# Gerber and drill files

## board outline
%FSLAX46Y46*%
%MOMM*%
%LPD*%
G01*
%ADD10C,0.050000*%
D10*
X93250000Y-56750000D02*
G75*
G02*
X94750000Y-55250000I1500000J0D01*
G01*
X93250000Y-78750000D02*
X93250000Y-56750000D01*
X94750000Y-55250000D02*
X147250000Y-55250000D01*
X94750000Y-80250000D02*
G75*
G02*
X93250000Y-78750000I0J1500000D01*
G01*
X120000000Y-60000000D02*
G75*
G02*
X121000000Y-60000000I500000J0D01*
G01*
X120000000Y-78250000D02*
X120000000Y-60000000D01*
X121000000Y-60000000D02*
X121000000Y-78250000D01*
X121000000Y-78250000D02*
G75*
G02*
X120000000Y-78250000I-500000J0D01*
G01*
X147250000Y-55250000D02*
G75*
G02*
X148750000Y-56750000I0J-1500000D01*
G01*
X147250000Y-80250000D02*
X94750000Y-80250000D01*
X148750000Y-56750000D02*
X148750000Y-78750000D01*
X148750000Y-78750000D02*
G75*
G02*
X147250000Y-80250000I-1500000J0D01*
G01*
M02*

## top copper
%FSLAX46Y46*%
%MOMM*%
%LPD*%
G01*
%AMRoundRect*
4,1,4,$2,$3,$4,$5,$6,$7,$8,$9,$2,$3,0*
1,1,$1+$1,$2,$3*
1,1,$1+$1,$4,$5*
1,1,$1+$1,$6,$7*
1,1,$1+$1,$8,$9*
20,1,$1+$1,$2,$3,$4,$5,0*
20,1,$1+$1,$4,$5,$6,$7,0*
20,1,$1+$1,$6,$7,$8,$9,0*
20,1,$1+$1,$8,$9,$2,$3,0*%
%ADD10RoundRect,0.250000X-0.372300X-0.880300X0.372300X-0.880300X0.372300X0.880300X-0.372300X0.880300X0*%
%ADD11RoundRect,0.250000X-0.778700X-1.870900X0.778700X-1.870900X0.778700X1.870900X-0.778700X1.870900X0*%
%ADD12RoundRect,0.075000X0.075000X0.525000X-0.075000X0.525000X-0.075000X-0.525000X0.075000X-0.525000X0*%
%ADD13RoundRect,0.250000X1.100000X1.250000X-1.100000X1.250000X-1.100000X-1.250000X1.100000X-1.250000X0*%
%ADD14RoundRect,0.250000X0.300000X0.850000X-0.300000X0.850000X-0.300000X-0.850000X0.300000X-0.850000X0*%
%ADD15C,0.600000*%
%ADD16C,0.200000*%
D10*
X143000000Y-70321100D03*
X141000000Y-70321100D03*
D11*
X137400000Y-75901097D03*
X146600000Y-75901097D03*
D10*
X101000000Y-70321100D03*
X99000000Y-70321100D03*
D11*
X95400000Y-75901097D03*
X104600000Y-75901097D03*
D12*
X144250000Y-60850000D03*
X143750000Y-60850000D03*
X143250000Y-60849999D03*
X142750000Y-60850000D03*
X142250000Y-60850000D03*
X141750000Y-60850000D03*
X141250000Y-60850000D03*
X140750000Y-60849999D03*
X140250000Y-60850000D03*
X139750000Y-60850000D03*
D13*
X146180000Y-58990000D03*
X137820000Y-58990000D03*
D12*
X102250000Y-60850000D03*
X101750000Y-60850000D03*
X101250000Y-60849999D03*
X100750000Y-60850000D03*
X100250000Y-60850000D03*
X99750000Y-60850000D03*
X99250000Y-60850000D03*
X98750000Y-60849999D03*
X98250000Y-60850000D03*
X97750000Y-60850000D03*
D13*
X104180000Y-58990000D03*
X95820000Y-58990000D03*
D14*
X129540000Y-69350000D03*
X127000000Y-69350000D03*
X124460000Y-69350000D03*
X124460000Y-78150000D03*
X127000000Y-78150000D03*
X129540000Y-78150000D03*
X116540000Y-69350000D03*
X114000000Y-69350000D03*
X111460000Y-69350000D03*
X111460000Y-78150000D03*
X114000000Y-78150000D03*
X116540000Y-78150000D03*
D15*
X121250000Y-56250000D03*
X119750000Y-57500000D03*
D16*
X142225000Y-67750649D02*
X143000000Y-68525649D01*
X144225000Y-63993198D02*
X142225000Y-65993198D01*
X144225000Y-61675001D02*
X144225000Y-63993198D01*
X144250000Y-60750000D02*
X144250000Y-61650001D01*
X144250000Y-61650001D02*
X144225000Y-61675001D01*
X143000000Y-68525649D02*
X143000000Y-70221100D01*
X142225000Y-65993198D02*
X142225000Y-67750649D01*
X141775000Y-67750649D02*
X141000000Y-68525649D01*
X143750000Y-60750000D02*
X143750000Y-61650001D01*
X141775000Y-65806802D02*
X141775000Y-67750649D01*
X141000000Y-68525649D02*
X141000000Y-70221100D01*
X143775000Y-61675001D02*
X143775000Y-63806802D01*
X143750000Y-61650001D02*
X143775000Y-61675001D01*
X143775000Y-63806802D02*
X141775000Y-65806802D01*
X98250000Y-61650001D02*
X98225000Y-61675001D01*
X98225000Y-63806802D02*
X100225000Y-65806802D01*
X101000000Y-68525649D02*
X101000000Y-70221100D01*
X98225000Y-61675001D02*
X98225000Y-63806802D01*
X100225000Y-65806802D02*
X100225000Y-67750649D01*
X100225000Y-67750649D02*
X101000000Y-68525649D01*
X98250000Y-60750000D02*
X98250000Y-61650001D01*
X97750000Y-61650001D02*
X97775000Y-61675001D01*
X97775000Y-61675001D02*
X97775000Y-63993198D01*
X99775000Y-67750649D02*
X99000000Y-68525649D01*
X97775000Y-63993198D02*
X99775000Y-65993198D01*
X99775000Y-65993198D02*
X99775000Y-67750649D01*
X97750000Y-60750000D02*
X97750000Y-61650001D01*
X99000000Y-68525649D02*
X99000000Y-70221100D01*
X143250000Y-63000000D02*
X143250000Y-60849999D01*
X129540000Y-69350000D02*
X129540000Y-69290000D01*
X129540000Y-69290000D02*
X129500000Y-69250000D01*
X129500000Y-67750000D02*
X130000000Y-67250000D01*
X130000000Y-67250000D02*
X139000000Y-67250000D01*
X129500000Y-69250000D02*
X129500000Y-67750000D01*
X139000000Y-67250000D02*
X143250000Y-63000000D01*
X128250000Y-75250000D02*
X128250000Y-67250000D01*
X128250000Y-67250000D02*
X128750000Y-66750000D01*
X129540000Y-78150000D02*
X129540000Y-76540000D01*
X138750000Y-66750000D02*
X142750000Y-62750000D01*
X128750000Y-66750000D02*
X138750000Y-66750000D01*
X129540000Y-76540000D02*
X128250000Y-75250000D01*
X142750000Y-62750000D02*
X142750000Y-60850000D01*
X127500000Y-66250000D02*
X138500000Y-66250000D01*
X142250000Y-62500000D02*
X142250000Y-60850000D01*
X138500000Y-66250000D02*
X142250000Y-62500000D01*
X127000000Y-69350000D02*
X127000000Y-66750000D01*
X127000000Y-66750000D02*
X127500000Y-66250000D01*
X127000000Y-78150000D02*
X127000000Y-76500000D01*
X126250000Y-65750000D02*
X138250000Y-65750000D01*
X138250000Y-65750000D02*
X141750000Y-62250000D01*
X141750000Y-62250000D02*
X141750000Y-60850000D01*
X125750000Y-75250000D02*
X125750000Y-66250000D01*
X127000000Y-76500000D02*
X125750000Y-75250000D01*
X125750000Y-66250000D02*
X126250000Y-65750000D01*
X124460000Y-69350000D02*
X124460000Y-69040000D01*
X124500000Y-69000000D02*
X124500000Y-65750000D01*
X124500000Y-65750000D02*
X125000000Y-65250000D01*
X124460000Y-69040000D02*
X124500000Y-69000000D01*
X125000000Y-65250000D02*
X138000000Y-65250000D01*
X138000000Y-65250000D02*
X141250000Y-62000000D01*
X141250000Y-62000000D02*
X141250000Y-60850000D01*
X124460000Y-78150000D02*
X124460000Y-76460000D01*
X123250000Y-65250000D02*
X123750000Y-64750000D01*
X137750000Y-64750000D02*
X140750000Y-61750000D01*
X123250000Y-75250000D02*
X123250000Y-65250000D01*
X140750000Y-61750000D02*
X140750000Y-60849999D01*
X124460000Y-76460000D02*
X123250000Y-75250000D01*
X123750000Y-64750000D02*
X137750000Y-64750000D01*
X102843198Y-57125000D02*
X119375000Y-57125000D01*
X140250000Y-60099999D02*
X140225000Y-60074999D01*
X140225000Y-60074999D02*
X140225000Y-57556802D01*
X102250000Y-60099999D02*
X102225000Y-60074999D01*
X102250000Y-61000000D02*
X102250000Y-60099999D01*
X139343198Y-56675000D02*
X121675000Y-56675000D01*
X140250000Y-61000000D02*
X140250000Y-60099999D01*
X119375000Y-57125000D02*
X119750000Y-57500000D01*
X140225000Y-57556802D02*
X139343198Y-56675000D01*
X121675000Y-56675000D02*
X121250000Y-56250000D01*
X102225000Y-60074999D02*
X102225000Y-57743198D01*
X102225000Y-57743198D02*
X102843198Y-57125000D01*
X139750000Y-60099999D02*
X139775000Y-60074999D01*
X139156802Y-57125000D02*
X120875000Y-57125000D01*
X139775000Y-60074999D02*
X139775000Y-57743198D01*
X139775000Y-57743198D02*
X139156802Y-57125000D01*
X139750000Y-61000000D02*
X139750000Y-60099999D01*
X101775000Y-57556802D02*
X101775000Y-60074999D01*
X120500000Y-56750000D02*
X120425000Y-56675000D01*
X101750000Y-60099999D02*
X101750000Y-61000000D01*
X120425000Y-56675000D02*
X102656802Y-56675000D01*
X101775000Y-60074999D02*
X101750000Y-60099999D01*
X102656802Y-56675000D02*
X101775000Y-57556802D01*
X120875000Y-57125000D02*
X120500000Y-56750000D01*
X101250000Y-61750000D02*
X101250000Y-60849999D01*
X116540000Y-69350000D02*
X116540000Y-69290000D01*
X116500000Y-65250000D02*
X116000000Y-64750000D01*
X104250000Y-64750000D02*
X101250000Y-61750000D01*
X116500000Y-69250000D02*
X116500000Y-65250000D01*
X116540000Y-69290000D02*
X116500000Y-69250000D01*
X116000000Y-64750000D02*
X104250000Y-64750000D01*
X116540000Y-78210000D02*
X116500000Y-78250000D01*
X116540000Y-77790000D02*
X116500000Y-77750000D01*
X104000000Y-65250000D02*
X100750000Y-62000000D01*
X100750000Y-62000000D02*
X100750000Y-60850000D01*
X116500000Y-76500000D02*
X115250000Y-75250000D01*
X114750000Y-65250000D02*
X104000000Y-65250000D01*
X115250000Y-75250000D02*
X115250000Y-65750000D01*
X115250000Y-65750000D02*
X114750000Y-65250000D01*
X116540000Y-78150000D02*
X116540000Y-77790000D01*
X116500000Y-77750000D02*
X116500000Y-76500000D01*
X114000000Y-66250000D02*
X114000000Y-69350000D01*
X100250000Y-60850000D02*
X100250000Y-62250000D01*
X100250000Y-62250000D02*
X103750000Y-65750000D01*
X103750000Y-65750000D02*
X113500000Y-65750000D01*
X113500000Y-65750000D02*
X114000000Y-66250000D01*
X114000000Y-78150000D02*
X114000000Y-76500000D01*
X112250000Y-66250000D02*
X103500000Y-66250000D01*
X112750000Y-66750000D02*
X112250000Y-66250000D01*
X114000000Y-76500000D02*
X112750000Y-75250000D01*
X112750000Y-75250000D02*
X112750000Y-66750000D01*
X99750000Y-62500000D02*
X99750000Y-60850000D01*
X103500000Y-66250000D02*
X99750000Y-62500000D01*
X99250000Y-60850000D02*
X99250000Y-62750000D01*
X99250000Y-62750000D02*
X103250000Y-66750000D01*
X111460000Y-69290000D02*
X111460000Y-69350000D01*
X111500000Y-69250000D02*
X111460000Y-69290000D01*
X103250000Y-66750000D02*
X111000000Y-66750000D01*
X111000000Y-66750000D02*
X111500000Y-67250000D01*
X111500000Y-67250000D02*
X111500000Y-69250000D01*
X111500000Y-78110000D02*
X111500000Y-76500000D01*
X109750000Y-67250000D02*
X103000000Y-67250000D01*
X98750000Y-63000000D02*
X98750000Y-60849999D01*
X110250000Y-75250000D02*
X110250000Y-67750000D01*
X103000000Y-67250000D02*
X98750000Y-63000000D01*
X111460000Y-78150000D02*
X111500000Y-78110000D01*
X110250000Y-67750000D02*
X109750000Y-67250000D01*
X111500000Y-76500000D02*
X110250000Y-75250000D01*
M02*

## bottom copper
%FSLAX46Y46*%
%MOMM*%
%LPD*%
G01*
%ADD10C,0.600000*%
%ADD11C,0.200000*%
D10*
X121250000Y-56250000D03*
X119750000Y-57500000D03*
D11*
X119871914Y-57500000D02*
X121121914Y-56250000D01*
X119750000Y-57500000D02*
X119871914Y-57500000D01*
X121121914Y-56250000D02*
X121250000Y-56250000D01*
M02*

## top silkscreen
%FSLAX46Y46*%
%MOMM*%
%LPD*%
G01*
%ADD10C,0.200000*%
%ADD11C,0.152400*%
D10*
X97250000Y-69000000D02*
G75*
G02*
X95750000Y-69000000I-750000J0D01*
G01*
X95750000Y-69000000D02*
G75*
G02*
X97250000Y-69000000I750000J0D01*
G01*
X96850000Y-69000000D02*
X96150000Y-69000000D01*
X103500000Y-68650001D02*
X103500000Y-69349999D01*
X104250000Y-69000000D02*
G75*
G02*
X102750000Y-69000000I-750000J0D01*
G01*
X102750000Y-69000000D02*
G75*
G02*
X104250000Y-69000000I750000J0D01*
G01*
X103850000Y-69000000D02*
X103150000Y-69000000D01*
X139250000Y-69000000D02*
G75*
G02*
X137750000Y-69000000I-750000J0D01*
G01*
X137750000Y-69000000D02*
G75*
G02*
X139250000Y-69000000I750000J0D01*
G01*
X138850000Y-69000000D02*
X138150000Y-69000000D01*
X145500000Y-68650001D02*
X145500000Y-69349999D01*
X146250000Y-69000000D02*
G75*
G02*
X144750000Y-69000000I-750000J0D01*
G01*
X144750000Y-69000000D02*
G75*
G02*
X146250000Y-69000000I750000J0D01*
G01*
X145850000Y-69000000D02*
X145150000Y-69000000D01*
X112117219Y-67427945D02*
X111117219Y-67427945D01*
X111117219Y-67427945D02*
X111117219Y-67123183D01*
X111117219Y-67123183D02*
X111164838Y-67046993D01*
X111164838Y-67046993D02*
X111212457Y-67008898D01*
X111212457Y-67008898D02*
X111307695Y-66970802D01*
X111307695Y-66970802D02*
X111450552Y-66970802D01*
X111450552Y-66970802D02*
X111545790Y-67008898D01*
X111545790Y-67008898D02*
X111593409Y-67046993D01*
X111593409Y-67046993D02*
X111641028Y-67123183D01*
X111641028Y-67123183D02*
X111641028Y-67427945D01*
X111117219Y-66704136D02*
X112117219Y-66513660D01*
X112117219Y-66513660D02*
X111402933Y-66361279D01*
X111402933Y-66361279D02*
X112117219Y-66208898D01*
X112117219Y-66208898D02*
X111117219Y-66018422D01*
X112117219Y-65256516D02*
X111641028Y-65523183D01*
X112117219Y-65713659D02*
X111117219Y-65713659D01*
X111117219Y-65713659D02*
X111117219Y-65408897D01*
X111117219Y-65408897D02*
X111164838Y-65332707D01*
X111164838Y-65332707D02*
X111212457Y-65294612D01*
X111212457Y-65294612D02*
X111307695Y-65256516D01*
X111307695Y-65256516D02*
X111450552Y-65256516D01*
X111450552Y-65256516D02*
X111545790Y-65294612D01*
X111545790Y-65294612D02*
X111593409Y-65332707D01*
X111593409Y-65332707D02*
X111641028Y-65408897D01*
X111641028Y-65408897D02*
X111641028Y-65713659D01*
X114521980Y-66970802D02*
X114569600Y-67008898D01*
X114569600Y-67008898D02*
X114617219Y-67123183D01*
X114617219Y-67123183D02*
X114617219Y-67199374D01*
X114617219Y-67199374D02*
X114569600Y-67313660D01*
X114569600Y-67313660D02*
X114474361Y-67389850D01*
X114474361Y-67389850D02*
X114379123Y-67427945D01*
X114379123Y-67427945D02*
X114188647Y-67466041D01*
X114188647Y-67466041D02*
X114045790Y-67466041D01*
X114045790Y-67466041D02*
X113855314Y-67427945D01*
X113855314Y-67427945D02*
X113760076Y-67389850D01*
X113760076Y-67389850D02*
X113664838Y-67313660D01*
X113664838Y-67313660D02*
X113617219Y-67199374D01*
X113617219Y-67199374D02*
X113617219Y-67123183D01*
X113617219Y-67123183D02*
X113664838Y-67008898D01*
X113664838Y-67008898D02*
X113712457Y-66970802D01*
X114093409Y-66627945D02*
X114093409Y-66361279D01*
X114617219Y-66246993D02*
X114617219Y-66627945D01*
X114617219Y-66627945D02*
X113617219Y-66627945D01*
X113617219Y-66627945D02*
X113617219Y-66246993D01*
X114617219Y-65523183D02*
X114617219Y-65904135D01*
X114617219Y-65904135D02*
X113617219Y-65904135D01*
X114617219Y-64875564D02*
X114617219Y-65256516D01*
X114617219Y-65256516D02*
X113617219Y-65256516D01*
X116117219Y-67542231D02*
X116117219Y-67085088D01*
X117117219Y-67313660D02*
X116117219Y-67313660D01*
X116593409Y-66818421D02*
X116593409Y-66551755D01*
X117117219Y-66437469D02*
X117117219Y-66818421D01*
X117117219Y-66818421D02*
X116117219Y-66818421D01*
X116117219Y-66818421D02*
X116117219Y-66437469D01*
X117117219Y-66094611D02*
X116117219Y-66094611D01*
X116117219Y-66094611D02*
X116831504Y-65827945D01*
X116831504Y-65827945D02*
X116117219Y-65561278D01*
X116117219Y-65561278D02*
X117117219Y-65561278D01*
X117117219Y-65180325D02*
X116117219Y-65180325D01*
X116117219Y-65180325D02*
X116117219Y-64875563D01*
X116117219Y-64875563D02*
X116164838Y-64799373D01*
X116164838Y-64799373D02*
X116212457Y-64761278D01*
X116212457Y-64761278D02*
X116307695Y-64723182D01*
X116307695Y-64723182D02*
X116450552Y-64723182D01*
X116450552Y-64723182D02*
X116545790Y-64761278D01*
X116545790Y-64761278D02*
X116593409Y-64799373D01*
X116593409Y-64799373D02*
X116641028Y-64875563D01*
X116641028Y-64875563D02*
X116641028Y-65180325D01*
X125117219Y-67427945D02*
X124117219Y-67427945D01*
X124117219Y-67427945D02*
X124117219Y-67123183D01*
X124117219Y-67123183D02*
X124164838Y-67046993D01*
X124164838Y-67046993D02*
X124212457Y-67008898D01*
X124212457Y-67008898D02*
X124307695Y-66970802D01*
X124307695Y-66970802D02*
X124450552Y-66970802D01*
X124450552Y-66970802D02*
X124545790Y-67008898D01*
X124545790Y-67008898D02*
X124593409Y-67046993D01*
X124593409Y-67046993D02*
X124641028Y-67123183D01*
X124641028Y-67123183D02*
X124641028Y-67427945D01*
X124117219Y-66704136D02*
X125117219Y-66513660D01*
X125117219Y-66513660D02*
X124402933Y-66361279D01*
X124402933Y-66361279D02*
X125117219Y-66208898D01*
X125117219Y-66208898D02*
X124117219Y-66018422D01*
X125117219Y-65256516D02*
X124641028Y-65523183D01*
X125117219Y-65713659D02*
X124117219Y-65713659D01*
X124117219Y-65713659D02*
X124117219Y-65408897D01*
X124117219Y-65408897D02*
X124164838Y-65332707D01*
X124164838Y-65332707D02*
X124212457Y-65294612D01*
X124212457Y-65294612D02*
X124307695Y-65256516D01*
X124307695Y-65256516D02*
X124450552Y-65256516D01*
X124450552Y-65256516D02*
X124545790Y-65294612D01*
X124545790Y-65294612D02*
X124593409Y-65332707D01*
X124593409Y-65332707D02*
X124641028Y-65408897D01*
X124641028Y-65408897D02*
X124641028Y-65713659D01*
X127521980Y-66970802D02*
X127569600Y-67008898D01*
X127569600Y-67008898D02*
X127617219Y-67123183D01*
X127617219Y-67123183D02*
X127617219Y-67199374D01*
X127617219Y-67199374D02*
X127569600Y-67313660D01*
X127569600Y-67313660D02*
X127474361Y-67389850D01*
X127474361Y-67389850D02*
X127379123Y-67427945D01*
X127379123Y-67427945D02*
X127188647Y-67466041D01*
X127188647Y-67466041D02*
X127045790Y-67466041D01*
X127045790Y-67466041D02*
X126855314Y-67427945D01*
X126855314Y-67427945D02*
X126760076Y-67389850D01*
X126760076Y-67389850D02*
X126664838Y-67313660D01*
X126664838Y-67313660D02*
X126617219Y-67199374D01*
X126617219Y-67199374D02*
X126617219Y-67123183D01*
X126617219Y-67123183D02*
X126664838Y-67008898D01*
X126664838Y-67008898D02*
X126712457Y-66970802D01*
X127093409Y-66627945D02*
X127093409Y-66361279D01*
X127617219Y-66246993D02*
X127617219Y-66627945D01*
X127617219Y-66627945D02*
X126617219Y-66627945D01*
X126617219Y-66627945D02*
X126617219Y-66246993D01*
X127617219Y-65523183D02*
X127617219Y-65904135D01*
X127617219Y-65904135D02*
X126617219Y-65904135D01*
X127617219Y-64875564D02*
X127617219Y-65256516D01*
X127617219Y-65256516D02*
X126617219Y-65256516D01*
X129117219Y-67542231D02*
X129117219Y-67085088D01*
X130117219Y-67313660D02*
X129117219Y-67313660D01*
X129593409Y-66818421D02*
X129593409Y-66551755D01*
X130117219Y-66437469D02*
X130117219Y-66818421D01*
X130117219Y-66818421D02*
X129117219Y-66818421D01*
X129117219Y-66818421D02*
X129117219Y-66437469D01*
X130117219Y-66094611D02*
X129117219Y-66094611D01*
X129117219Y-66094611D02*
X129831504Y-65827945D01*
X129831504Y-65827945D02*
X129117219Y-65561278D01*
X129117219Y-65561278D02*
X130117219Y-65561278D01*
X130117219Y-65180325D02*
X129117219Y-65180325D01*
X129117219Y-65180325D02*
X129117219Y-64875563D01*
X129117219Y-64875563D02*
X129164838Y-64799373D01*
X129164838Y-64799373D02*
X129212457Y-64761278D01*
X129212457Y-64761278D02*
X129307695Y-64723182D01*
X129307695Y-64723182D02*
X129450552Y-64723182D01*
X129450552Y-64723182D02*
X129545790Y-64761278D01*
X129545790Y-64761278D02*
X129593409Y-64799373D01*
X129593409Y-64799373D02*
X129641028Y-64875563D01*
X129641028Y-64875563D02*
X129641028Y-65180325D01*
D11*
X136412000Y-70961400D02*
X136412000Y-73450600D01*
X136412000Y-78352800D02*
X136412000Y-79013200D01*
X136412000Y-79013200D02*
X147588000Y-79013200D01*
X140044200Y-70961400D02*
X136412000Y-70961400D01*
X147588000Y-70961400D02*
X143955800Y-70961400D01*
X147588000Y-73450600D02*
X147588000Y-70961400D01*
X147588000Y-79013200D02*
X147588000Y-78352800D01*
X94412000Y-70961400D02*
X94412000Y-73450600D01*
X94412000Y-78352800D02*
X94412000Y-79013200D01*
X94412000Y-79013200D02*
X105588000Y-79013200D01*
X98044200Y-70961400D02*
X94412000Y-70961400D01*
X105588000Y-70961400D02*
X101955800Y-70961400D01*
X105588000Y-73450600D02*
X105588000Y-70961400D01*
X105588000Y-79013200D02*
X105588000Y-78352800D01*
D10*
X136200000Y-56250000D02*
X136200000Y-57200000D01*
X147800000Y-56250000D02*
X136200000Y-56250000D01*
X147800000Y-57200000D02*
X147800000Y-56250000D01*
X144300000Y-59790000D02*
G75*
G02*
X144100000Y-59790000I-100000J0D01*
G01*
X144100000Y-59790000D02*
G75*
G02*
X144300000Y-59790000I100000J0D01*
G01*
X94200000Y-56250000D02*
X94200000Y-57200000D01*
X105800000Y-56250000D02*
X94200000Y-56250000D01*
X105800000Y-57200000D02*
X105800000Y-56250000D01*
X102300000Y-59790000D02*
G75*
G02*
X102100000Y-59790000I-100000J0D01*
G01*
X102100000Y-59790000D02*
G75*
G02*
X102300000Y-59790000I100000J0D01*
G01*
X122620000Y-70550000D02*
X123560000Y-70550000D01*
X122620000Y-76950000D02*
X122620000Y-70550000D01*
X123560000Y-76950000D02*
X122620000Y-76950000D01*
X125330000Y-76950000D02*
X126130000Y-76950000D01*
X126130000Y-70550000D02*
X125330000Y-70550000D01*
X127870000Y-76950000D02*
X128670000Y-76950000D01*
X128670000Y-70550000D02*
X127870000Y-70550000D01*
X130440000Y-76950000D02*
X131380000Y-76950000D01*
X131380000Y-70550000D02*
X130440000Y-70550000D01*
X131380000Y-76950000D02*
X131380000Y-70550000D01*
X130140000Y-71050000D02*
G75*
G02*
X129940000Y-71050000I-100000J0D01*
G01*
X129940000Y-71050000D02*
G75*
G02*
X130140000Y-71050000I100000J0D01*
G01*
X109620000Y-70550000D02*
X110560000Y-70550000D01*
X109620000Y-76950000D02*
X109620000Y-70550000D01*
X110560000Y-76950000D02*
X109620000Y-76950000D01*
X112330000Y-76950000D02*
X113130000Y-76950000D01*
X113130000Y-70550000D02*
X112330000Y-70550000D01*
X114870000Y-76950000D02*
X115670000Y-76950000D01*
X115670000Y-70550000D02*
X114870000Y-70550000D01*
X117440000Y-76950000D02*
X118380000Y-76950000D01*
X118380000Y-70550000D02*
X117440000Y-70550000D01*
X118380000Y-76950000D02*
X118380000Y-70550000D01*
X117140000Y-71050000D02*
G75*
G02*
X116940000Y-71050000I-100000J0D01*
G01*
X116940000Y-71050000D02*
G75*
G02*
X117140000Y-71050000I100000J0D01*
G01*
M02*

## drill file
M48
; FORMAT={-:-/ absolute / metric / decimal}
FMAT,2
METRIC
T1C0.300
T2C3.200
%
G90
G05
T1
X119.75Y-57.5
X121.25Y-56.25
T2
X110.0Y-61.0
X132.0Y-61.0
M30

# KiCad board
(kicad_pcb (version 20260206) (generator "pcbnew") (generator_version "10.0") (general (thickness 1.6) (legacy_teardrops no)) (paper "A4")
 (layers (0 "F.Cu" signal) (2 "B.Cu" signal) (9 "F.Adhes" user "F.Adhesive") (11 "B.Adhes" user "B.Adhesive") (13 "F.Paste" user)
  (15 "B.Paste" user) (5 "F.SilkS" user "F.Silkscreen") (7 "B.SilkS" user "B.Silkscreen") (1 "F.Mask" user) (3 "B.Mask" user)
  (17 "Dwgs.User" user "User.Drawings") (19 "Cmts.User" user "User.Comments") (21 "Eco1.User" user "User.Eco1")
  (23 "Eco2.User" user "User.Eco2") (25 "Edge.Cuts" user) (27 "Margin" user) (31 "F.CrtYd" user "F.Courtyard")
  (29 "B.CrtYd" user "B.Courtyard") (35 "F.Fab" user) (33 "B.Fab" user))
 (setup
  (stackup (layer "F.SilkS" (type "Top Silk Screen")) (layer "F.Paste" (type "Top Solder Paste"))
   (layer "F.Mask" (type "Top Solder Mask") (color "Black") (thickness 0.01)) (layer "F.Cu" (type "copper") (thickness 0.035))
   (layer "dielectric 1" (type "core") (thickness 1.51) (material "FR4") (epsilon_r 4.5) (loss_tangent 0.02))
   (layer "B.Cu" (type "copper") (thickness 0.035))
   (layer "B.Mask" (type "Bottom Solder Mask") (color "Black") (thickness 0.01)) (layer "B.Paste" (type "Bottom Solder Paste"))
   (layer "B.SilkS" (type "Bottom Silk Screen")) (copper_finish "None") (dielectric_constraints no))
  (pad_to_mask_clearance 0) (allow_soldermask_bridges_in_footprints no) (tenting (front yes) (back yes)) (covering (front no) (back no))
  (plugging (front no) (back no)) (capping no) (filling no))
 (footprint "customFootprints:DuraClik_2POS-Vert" (layer "F.Cu") (at 142 75)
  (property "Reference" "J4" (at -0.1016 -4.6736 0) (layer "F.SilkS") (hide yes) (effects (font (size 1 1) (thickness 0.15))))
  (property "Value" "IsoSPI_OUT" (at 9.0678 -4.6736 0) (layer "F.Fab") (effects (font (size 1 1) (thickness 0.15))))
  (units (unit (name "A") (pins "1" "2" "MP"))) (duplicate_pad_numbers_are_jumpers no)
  (fp_line (start -5.588 -4.0386) (end -5.588 -1.5494) (stroke (width 0.1524) (type solid)) (layer "F.SilkS"))
  (fp_line (start -5.588 3.3528) (end -5.588 4.0132) (stroke (width 0.1524) (type solid)) (layer "F.SilkS"))
  (fp_line (start -5.588 4.0132) (end 5.588 4.0132) (stroke (width 0.1524) (type solid)) (layer "F.SilkS"))
  (fp_line (start -1.9558 -4.0386) (end -5.588 -4.0386) (stroke (width 0.1524) (type solid)) (layer "F.SilkS"))
  (fp_line (start 5.588 -4.0386) (end 1.9558 -4.0386) (stroke (width 0.1524) (type solid)) (layer "F.SilkS"))
  (fp_line (start 5.588 -1.5494) (end 5.588 -4.0386) (stroke (width 0.1524) (type solid)) (layer "F.SilkS"))
  (fp_line (start 5.588 4.0132) (end 5.588 3.3528) (stroke (width 0.1524) (type solid)) (layer "F.SilkS"))
  (pad "1" smd roundrect (at 1 -4.6789) (size 1.2446 2.2606) (layers "F.Cu" "F.Mask" "F.Paste") (roundrect_rratio 0.2008677487)
   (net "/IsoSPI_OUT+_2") (solder_mask_margin 0))
  (pad "2" smd roundrect (at -1 -4.6789) (size 1.2446 2.2606) (layers "F.Cu" "F.Mask" "F.Paste") (roundrect_rratio 0.2008677487)
   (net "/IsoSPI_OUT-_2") (solder_mask_margin 0))
  (pad "MP" smd roundrect (at -4.6 0.901097) (size 2.0574 4.2418) (layers "F.Cu" "F.Mask" "F.Paste") (roundrect_rratio 0.1215125887)
   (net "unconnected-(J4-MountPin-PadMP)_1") (solder_mask_margin 0))
  (pad "MP" smd roundrect (at 4.6 0.901097) (size 2.0574 4.2418) (layers "F.Cu" "F.Mask" "F.Paste") (roundrect_rratio 0.1215125887)
   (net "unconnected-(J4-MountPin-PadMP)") (solder_mask_margin 0)))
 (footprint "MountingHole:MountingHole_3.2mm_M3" (layer "F.Cu") (at 110 61)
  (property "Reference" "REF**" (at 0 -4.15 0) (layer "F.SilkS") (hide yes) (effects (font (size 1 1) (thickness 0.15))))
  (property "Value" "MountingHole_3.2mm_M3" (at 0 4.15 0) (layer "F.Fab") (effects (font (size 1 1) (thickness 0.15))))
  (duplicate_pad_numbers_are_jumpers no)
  (pad "" np_thru_hole circle (at 0 0) (size 3.2 3.2) (drill 3.2) (layers "*.Cu" "*.Mask")))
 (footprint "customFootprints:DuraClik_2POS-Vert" (layer "F.Cu") (at 100 75)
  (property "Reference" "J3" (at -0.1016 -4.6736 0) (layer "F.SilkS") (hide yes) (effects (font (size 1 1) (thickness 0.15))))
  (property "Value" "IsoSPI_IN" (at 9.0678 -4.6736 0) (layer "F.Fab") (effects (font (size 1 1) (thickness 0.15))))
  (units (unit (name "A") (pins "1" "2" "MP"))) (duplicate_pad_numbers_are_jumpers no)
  (fp_line (start -5.588 -4.0386) (end -5.588 -1.5494) (stroke (width 0.1524) (type solid)) (layer "F.SilkS"))
  (fp_line (start -5.588 3.3528) (end -5.588 4.0132) (stroke (width 0.1524) (type solid)) (layer "F.SilkS"))
  (fp_line (start -5.588 4.0132) (end 5.588 4.0132) (stroke (width 0.1524) (type solid)) (layer "F.SilkS"))
  (fp_line (start -1.9558 -4.0386) (end -5.588 -4.0386) (stroke (width 0.1524) (type solid)) (layer "F.SilkS"))
  (fp_line (start 5.588 -4.0386) (end 1.9558 -4.0386) (stroke (width 0.1524) (type solid)) (layer "F.SilkS"))
  (fp_line (start 5.588 -1.5494) (end 5.588 -4.0386) (stroke (width 0.1524) (type solid)) (layer "F.SilkS"))
  (fp_line (start 5.588 4.0132) (end 5.588 3.3528) (stroke (width 0.1524) (type solid)) (layer "F.SilkS"))
  (pad "1" smd roundrect (at 1 -4.6789) (size 1.2446 2.2606) (layers "F.Cu" "F.Mask" "F.Paste") (roundrect_rratio 0.2008677487)
   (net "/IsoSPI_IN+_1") (solder_mask_margin 0))
  (pad "2" smd roundrect (at -1 -4.6789) (size 1.2446 2.2606) (layers "F.Cu" "F.Mask" "F.Paste") (roundrect_rratio 0.2008677487)
   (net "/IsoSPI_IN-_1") (solder_mask_margin 0))
  (pad "MP" smd roundrect (at -4.6 0.901097) (size 2.0574 4.2418) (layers "F.Cu" "F.Mask" "F.Paste") (roundrect_rratio 0.1215125887)
   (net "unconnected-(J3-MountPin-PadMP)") (solder_mask_margin 0))
  (pad "MP" smd roundrect (at 4.6 0.901097) (size 2.0574 4.2418) (layers "F.Cu" "F.Mask" "F.Paste") (roundrect_rratio 0.1215125887)
   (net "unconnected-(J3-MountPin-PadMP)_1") (solder_mask_margin 0)))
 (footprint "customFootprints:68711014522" (layer "F.Cu") (at 142 58.5 180)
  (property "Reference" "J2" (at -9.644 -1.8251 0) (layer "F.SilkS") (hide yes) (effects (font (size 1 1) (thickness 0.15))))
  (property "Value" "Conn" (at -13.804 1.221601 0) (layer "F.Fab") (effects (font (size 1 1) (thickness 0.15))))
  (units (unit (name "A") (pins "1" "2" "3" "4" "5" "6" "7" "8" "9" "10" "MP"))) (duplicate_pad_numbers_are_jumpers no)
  (fp_line (start 5.8 2.25) (end 5.8 1.3) (stroke (width 0.2) (type solid)) (layer "F.SilkS"))
  (fp_line (start -5.8 2.25) (end 5.8 2.25) (stroke (width 0.2) (type solid)) (layer "F.SilkS"))
  (fp_line (start -5.8 1.3) (end -5.8 2.25) (stroke (width 0.2) (type solid)) (layer "F.SilkS"))
  (fp_circle (center -2.2 -1.29) (end -2.1 -1.29) (stroke (width 0.2) (type solid)) (fill no) (layer "F.SilkS"))
  (pad "1" smd roundrect (at -2.25 -2.35 180) (size 0.3 1.2) (layers "F.Cu" "F.Mask" "F.Paste") (roundrect_rratio 0.25)
   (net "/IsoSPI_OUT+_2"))
  (pad "2" smd roundrect (at -1.75 -2.35 180) (size 0.3 1.2) (layers "F.Cu" "F.Mask" "F.Paste") (roundrect_rratio 0.25)
   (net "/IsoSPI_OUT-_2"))
  (pad "3" smd roundrect (at -1.25 -2.349999 180) (size 0.3 1.2) (layers "F.Cu" "F.Mask" "F.Paste") (roundrect_rratio 0.25)
   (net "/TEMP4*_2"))
  (pad "4" smd roundrect (at -0.75 -2.35 180) (size 0.3 1.2) (layers "F.Cu" "F.Mask" "F.Paste") (roundrect_rratio 0.25) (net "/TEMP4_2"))
  (pad "5" smd roundrect (at -0.25 -2.35 180) (size 0.3 1.2) (layers "F.Cu" "F.Mask" "F.Paste") (roundrect_rratio 0.25) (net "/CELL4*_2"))
  (pad "6" smd roundrect (at 0.25 -2.35 180) (size 0.3 1.2) (layers "F.Cu" "F.Mask" "F.Paste") (roundrect_rratio 0.25) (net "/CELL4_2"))
  (pad "7" smd roundrect (at 0.75 -2.35 180) (size 0.3 1.2) (layers "F.Cu" "F.Mask" "F.Paste") (roundrect_rratio 0.25) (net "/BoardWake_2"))
  (pad "8" smd roundrect (at 1.25 -2.349999 180) (size 0.3 1.2) (layers "F.Cu" "F.Mask" "F.Paste") (roundrect_rratio 0.25) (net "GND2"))
  (pad "9" smd roundrect (at 1.75 -2.35 180) (size 0.3 1.2) (layers "F.Cu" "F.Mask" "F.Paste") (roundrect_rratio 0.25) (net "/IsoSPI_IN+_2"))
  (pad "10" smd roundrect (at 2.25 -2.35 180) (size 0.3 1.2) (layers "F.Cu" "F.Mask" "F.Paste") (roundrect_rratio 0.25)
   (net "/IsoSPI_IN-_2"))
  (pad "MP" smd roundrect (at -4.18 -0.49 180) (size 2.7 3) (layers "F.Cu" "F.Mask" "F.Paste") (roundrect_rratio 0.09259259259)
   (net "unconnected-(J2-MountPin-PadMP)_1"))
  (pad "MP" smd roundrect (at 4.18 -0.49 180) (size 2.7 3) (layers "F.Cu" "F.Mask" "F.Paste") (roundrect_rratio 0.09259259259)
   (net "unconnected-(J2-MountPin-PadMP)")))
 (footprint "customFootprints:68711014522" (layer "F.Cu") (at 100 58.5 180)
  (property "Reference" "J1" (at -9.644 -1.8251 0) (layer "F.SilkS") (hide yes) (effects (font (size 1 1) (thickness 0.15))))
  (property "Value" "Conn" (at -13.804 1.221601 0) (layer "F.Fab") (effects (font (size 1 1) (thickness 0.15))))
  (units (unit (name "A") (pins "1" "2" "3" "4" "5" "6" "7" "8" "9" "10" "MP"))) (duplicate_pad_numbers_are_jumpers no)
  (fp_line (start 5.8 2.25) (end 5.8 1.3) (stroke (width 0.2) (type solid)) (layer "F.SilkS"))
  (fp_line (start -5.8 2.25) (end 5.8 2.25) (stroke (width 0.2) (type solid)) (layer "F.SilkS"))
  (fp_line (start -5.8 1.3) (end -5.8 2.25) (stroke (width 0.2) (type solid)) (layer "F.SilkS"))
  (fp_circle (center -2.2 -1.29) (end -2.1 -1.29) (stroke (width 0.2) (type solid)) (fill no) (layer "F.SilkS"))
  (pad "1" smd roundrect (at -2.25 -2.35 180) (size 0.3 1.2) (layers "F.Cu" "F.Mask" "F.Paste") (roundrect_rratio 0.25)
   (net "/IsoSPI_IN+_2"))
  (pad "2" smd roundrect (at -1.75 -2.35 180) (size 0.3 1.2) (layers "F.Cu" "F.Mask" "F.Paste") (roundrect_rratio 0.25)
   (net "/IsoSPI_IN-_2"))
  (pad "3" smd roundrect (at -1.25 -2.349999 180) (size 0.3 1.2) (layers "F.Cu" "F.Mask" "F.Paste") (roundrect_rratio 0.25)
   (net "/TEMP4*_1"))
  (pad "4" smd roundrect (at -0.75 -2.35 180) (size 0.3 1.2) (layers "F.Cu" "F.Mask" "F.Paste") (roundrect_rratio 0.25) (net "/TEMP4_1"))
  (pad "5" smd roundrect (at -0.25 -2.35 180) (size 0.3 1.2) (layers "F.Cu" "F.Mask" "F.Paste") (roundrect_rratio 0.25) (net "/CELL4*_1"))
  (pad "6" smd roundrect (at 0.25 -2.35 180) (size 0.3 1.2) (layers "F.Cu" "F.Mask" "F.Paste") (roundrect_rratio 0.25) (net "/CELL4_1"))
  (pad "7" smd roundrect (at 0.75 -2.35 180) (size 0.3 1.2) (layers "F.Cu" "F.Mask" "F.Paste") (roundrect_rratio 0.25) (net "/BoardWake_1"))
  (pad "8" smd roundrect (at 1.25 -2.349999 180) (size 0.3 1.2) (layers "F.Cu" "F.Mask" "F.Paste") (roundrect_rratio 0.25) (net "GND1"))
  (pad "9" smd roundrect (at 1.75 -2.35 180) (size 0.3 1.2) (layers "F.Cu" "F.Mask" "F.Paste") (roundrect_rratio 0.25) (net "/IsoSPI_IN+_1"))
  (pad "10" smd roundrect (at 2.25 -2.35 180) (size 0.3 1.2) (layers "F.Cu" "F.Mask" "F.Paste") (roundrect_rratio 0.25)
   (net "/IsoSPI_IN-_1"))
  (pad "MP" smd roundrect (at -4.18 -0.49 180) (size 2.7 3) (layers "F.Cu" "F.Mask" "F.Paste") (roundrect_rratio 0.09259259259)
   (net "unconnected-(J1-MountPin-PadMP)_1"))
  (pad "MP" smd roundrect (at 4.18 -0.49 180) (size 2.7 3) (layers "F.Cu" "F.Mask" "F.Paste") (roundrect_rratio 0.09259259259)
   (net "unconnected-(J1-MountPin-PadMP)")))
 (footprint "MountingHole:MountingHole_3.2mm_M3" (layer "F.Cu") (at 132 61)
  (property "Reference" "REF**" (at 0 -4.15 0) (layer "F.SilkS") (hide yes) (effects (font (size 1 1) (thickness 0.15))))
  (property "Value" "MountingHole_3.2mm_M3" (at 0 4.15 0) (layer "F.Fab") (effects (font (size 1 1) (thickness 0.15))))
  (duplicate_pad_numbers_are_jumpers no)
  (pad "" np_thru_hole circle (at 0 0) (size 3.2 3.2) (drill 3.2) (layers "*.Cu" "*.Mask")))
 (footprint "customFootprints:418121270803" (layer "F.Cu") (at 127 73.75 180)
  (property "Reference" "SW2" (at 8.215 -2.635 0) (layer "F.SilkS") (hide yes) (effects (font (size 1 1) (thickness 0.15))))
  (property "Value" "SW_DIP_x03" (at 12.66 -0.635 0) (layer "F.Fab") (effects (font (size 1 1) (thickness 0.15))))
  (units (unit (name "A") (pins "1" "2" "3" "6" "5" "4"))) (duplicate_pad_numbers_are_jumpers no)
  (fp_line (start 4.38 3.2) (end 3.44 3.2) (stroke (width 0.2) (type solid)) (layer "F.SilkS"))
  (fp_line (start 4.38 -3.2) (end 4.38 3.2) (stroke (width 0.2) (type solid)) (layer "F.SilkS"))
  (fp_line (start 3.44 -3.2) (end 4.38 -3.2) (stroke (width 0.2) (type solid)) (layer "F.SilkS"))
  (fp_line (start 1.67 -3.2) (end 0.87 -3.2) (stroke (width 0.2) (type solid)) (layer "F.SilkS"))
  (fp_line (start 0.87 3.2) (end 1.67 3.2) (stroke (width 0.2) (type solid)) (layer "F.SilkS"))
  (fp_line (start -0.87 -3.2) (end -1.67 -3.2) (stroke (width 0.2) (type solid)) (layer "F.SilkS"))
  (fp_line (start -1.67 3.2) (end -0.87 3.2) (stroke (width 0.2) (type solid)) (layer "F.SilkS"))
  (fp_line (start -3.44 -3.2) (end -4.38 -3.2) (stroke (width 0.2) (type solid)) (layer "F.SilkS"))
  (fp_line (start -4.38 3.2) (end -3.44 3.2) (stroke (width 0.2) (type solid)) (layer "F.SilkS"))
  (fp_line (start -4.38 -3.2) (end -4.38 3.2) (stroke (width 0.2) (type solid)) (layer "F.SilkS"))
  (fp_circle (center -3.04 2.7) (end -2.94 2.7) (stroke (width 0.2) (type solid)) (fill no) (layer "F.SilkS"))
  (pad "1" smd roundrect (at -2.54 4.4 180) (size 1.1 2.2) (layers "F.Cu" "F.Mask" "F.Paste") (roundrect_rratio 0.2272727273)
   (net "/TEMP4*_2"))
  (pad "2" smd roundrect (at 0 4.4 180) (size 1.1 2.2) (layers "F.Cu" "F.Mask" "F.Paste") (roundrect_rratio 0.2272727273) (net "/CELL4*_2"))
  (pad "3" smd roundrect (at 2.54 4.4 180) (size 1.1 2.2) (layers "F.Cu" "F.Mask" "F.Paste") (roundrect_rratio 0.2272727273)
   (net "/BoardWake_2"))
  (pad "4" smd roundrect (at 2.54 -4.4 180) (size 1.1 2.2) (layers "F.Cu" "F.Mask" "F.Paste") (roundrect_rratio 0.2272727273) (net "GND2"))
  (pad "5" smd roundrect (at 0 -4.4 180) (size 1.1 2.2) (layers "F.Cu" "F.Mask" "F.Paste") (roundrect_rratio 0.2272727273) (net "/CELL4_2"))
  (pad "6" smd roundrect (at -2.54 -4.4 180) (size 1.1 2.2) (layers "F.Cu" "F.Mask" "F.Paste") (roundrect_rratio 0.2272727273)
   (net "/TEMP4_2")))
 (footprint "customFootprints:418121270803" (layer "F.Cu") (at 114 73.75 180)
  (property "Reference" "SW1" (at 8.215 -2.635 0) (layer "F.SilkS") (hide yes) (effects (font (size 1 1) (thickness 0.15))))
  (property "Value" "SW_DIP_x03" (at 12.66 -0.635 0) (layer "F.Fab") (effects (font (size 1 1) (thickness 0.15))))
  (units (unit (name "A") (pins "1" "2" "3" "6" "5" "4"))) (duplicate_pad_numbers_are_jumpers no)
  (fp_line (start 4.38 3.2) (end 3.44 3.2) (stroke (width 0.2) (type solid)) (layer "F.SilkS"))
  (fp_line (start 4.38 -3.2) (end 4.38 3.2) (stroke (width 0.2) (type solid)) (layer "F.SilkS"))
  (fp_line (start 3.44 -3.2) (end 4.38 -3.2) (stroke (width 0.2) (type solid)) (layer "F.SilkS"))
  (fp_line (start 1.67 -3.2) (end 0.87 -3.2) (stroke (width 0.2) (type solid)) (layer "F.SilkS"))
  (fp_line (start 0.87 3.2) (end 1.67 3.2) (stroke (width 0.2) (type solid)) (layer "F.SilkS"))
  (fp_line (start -0.87 -3.2) (end -1.67 -3.2) (stroke (width 0.2) (type solid)) (layer "F.SilkS"))
  (fp_line (start -1.67 3.2) (end -0.87 3.2) (stroke (width 0.2) (type solid)) (layer "F.SilkS"))
  (fp_line (start -3.44 -3.2) (end -4.38 -3.2) (stroke (width 0.2) (type solid)) (layer "F.SilkS"))
  (fp_line (start -4.38 3.2) (end -3.44 3.2) (stroke (width 0.2) (type solid)) (layer "F.SilkS"))
  (fp_line (start -4.38 -3.2) (end -4.38 3.2) (stroke (width 0.2) (type solid)) (layer "F.SilkS"))
  (fp_circle (center -3.04 2.7) (end -2.94 2.7) (stroke (width 0.2) (type solid)) (fill no) (layer "F.SilkS"))
  (pad "1" smd roundrect (at -2.54 4.4 180) (size 1.1 2.2) (layers "F.Cu" "F.Mask" "F.Paste") (roundrect_rratio 0.2272727273)
   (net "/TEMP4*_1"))
  (pad "2" smd roundrect (at 0 4.4 180) (size 1.1 2.2) (layers "F.Cu" "F.Mask" "F.Paste") (roundrect_rratio 0.2272727273) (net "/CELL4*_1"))
  (pad "3" smd roundrect (at 2.54 4.4 180) (size 1.1 2.2) (layers "F.Cu" "F.Mask" "F.Paste") (roundrect_rratio 0.2272727273)
   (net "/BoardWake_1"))
  (pad "4" smd roundrect (at 2.54 -4.4 180) (size 1.1 2.2) (layers "F.Cu" "F.Mask" "F.Paste") (roundrect_rratio 0.2272727273) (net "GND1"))
  (pad "5" smd roundrect (at 0 -4.4 180) (size 1.1 2.2) (layers "F.Cu" "F.Mask" "F.Paste") (roundrect_rratio 0.2272727273) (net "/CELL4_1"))
  (pad "6" smd roundrect (at -2.54 -4.4 180) (size 1.1 2.2) (layers "F.Cu" "F.Mask" "F.Paste") (roundrect_rratio 0.2272727273)
   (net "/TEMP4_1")))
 (gr_circle (center 96.5 69) (end 97.25 69) (stroke (width 0.2) (type default)) (fill no) (layer "F.SilkS"))
 (gr_line (start 96.85 69) (end 96.15 69) (stroke (width 0.2) (type solid)) (layer "F.SilkS"))
 (gr_line (start 103.5 68.650001) (end 103.5 69.349999) (stroke (width 0.2) (type solid)) (layer "F.SilkS"))
 (gr_circle (center 103.5 69) (end 104.25 69) (stroke (width 0.2) (type default)) (fill no) (layer "F.SilkS"))
 (gr_line (start 103.85 69) (end 103.15 69) (stroke (width 0.2) (type solid)) (layer "F.SilkS"))
 (gr_circle (center 138.5 69) (end 139.25 69) (stroke (width 0.2) (type default)) (fill no) (layer "F.SilkS"))
 (gr_line (start 138.85 69) (end 138.15 69) (stroke (width 0.2) (type solid)) (layer "F.SilkS"))
 (gr_line (start 145.5 68.650001) (end 145.5 69.349999) (stroke (width 0.2) (type solid)) (layer "F.SilkS"))
 (gr_circle (center 145.5 69) (end 146.25 69) (stroke (width 0.2) (type default)) (fill no) (layer "F.SilkS"))
 (gr_line (start 145.85 69) (end 145.15 69) (stroke (width 0.2) (type solid)) (layer "F.SilkS"))
 (gr_arc (start 93.25 56.75) (mid 93.68934 55.68934) (end 94.75 55.25) (stroke (width 0.05) (type default)) (layer "Edge.Cuts"))
 (gr_line (start 93.25 78.75) (end 93.25 56.75) (stroke (width 0.05) (type default)) (layer "Edge.Cuts"))
 (gr_line (start 94.75 55.25) (end 147.25 55.25) (stroke (width 0.05) (type default)) (layer "Edge.Cuts"))
 (gr_arc (start 94.75 80.25) (mid 93.68934 79.81066) (end 93.25 78.75) (stroke (width 0.05) (type default)) (layer "Edge.Cuts"))
 (gr_arc (start 120 60) (mid 120.5 59.5) (end 121 60) (stroke (width 0.05) (type default)) (layer "Edge.Cuts"))
 (gr_line (start 120 78.25) (end 120 60) (stroke (width 0.05) (type default)) (layer "Edge.Cuts"))
 (gr_line (start 121 60) (end 121 78.25) (stroke (width 0.05) (type default)) (layer "Edge.Cuts"))
 (gr_arc (start 121 78.25) (mid 120.5 78.75) (end 120 78.25) (stroke (width 0.05) (type default)) (layer "Edge.Cuts"))
 (gr_arc (start 147.25 55.25) (mid 148.31066 55.68934) (end 148.75 56.75) (stroke (width 0.05) (type default)) (layer "Edge.Cuts"))
 (gr_line (start 147.25 80.25) (end 94.75 80.25) (stroke (width 0.05) (type default)) (layer "Edge.Cuts"))
 (gr_line (start 148.75 56.75) (end 148.75 78.75) (stroke (width 0.05) (type default)) (layer "Edge.Cuts"))
 (gr_arc (start 148.75 78.75) (mid 148.31066 79.81066) (end 147.25 80.25) (stroke (width 0.05) (type default)) (layer "Edge.Cuts"))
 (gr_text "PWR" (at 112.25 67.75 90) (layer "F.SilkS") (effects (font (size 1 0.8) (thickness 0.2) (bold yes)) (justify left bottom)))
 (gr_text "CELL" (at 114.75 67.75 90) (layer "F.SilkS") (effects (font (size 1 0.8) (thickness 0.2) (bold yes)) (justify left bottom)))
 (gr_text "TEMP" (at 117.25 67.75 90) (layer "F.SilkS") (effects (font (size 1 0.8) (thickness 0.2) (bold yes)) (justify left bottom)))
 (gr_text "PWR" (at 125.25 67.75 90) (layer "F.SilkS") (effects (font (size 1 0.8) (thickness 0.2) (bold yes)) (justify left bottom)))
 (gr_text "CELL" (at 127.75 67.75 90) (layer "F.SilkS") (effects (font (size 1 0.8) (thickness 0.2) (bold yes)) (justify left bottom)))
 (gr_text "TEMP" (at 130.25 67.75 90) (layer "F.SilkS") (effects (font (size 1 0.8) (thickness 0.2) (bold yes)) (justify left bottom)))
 (segment (start 142.225 67.750649) (end 143 68.525649) (width 0.2) (layer "F.Cu") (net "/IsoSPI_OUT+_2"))
 (segment (start 144.225 63.993198) (end 142.225 65.993198) (width 0.2) (layer "F.Cu") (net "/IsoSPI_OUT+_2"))
 (segment (start 144.225 61.675001) (end 144.225 63.993198) (width 0.2) (layer "F.Cu") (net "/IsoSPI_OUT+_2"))
 (segment (start 144.25 60.75) (end 144.25 61.650001) (width 0.2) (layer "F.Cu") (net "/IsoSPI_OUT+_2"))
 (segment (start 144.25 61.650001) (end 144.225 61.675001) (width 0.2) (layer "F.Cu") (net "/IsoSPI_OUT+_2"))
 (segment (start 143 68.525649) (end 143 70.2211) (width 0.2) (layer "F.Cu") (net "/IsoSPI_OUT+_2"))
 (segment (start 142.225 65.993198) (end 142.225 67.750649) (width 0.2) (layer "F.Cu") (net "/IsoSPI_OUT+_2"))
 (segment (start 141.775 67.750649) (end 141 68.525649) (width 0.2) (layer "F.Cu") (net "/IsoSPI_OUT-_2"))
 (segment (start 143.75 60.75) (end 143.75 61.650001) (width 0.2) (layer "F.Cu") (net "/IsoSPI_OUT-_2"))
 (segment (start 141.775 65.806802) (end 141.775 67.750649) (width 0.2) (layer "F.Cu") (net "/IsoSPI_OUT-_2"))
 (segment (start 141 68.525649) (end 141 70.2211) (width 0.2) (layer "F.Cu") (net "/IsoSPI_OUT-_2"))
 (segment (start 143.775 61.675001) (end 143.775 63.806802) (width 0.2) (layer "F.Cu") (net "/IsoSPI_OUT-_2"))
 (segment (start 143.75 61.650001) (end 143.775 61.675001) (width 0.2) (layer "F.Cu") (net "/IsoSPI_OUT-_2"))
 (segment (start 143.775 63.806802) (end 141.775 65.806802) (width 0.2) (layer "F.Cu") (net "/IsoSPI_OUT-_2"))
 (segment (start 98.25 61.650001) (end 98.225 61.675001) (width 0.2) (layer "F.Cu") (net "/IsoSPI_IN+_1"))
 (segment (start 98.225 63.806802) (end 100.225 65.806802) (width 0.2) (layer "F.Cu") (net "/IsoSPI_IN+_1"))
 (segment (start 101 68.525649) (end 101 70.2211) (width 0.2) (layer "F.Cu") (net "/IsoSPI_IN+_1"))
 (segment (start 98.225 61.675001) (end 98.225 63.806802) (width 0.2) (layer "F.Cu") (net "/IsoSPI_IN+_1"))
 (segment (start 100.225 65.806802) (end 100.225 67.750649) (width 0.2) (layer "F.Cu") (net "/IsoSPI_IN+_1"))
 (segment (start 100.225 67.750649) (end 101 68.525649) (width 0.2) (layer "F.Cu") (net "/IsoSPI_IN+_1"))
 (segment (start 98.25 60.75) (end 98.25 61.650001) (width 0.2) (layer "F.Cu") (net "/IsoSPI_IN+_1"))
 (segment (start 97.75 61.650001) (end 97.775 61.675001) (width 0.2) (layer "F.Cu") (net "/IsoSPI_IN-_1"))
 (segment (start 97.775 61.675001) (end 97.775 63.993198) (width 0.2) (layer "F.Cu") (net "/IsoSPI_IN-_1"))
 (segment (start 99.775 67.750649) (end 99 68.525649) (width 0.2) (layer "F.Cu") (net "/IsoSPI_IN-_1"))
 (segment (start 97.775 63.993198) (end 99.775 65.993198) (width 0.2) (layer "F.Cu") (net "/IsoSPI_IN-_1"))
 (segment (start 99.775 65.993198) (end 99.775 67.750649) (width 0.2) (layer "F.Cu") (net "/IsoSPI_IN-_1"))
 (segment (start 97.75 60.75) (end 97.75 61.650001) (width 0.2) (layer "F.Cu") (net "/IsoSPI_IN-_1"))
 (segment (start 99 68.525649) (end 99 70.2211) (width 0.2) (layer "F.Cu") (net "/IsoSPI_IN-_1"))
 (segment (start 143.25 63) (end 143.25 60.849999) (width 0.2) (layer "F.Cu") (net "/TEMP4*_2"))
 (segment (start 129.54 69.35) (end 129.54 69.29) (width 0.2) (layer "F.Cu") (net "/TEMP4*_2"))
 (segment (start 129.54 69.29) (end 129.5 69.25) (width 0.2) (layer "F.Cu") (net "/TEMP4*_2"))
 (segment (start 129.5 67.75) (end 130 67.25) (width 0.2) (layer "F.Cu") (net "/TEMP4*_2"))
 (segment (start 130 67.25) (end 139 67.25) (width 0.2) (layer "F.Cu") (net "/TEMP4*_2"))
 (segment (start 129.5 69.25) (end 129.5 67.75) (width 0.2) (layer "F.Cu") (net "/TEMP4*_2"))
 (segment (start 139 67.25) (end 143.25 63) (width 0.2) (layer "F.Cu") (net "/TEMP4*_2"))
 (segment (start 128.25 75.25) (end 128.25 67.25) (width 0.2) (layer "F.Cu") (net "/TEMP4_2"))
 (segment (start 128.25 67.25) (end 128.75 66.75) (width 0.2) (layer "F.Cu") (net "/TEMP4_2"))
 (segment (start 129.54 78.15) (end 129.54 76.54) (width 0.2) (layer "F.Cu") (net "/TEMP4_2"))
 (segment (start 138.75 66.75) (end 142.75 62.75) (width 0.2) (layer "F.Cu") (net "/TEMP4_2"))
 (segment (start 128.75 66.75) (end 138.75 66.75) (width 0.2) (layer "F.Cu") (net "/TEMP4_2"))
 (segment (start 129.54 76.54) (end 128.25 75.25) (width 0.2) (layer "F.Cu") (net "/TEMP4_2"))
 (segment (start 142.75 62.75) (end 142.75 60.85) (width 0.2) (layer "F.Cu") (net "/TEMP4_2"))
 (segment (start 127.5 66.25) (end 138.5 66.25) (width 0.2) (layer "F.Cu") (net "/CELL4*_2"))
 (segment (start 142.25 62.5) (end 142.25 60.85) (width 0.2) (layer "F.Cu") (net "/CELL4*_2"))
 (segment (start 138.5 66.25) (end 142.25 62.5) (width 0.2) (layer "F.Cu") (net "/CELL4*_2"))
 (segment (start 127 69.35) (end 127 66.75) (width 0.2) (layer "F.Cu") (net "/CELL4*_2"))
 (segment (start 127 66.75) (end 127.5 66.25) (width 0.2) (layer "F.Cu") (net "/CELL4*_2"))
 (segment (start 127 78.15) (end 127 76.5) (width 0.2) (layer "F.Cu") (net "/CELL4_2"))
 (segment (start 126.25 65.75) (end 138.25 65.75) (width 0.2) (layer "F.Cu") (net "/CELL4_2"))
 (segment (start 138.25 65.75) (end 141.75 62.25) (width 0.2) (layer "F.Cu") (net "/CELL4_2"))
 (segment (start 141.75 62.25) (end 141.75 60.85) (width 0.2) (layer "F.Cu") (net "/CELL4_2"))
 (segment (start 125.75 75.25) (end 125.75 66.25) (width 0.2) (layer "F.Cu") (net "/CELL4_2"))
 (segment (start 127 76.5) (end 125.75 75.25) (width 0.2) (layer "F.Cu") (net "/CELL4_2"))
 (segment (start 125.75 66.25) (end 126.25 65.75) (width 0.2) (layer "F.Cu") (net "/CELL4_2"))
 (segment (start 124.46 69.35) (end 124.46 69.04) (width 0.2) (layer "F.Cu") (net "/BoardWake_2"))
 (segment (start 124.5 69) (end 124.5 65.75) (width 0.2) (layer "F.Cu") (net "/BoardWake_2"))
 (segment (start 124.5 65.75) (end 125 65.25) (width 0.2) (layer "F.Cu") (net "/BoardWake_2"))
 (segment (start 124.46 69.04) (end 124.5 69) (width 0.2) (layer "F.Cu") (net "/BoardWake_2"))
 (segment (start 125 65.25) (end 138 65.25) (width 0.2) (layer "F.Cu") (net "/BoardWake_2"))
 (segment (start 138 65.25) (end 141.25 62) (width 0.2) (layer "F.Cu") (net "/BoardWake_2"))
 (segment (start 141.25 62) (end 141.25 60.85) (width 0.2) (layer "F.Cu") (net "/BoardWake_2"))
 (segment (start 124.46 78.15) (end 124.46 76.46) (width 0.2) (layer "F.Cu") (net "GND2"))
 (segment (start 123.25 65.25) (end 123.75 64.75) (width 0.2) (layer "F.Cu") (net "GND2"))
 (segment (start 137.75 64.75) (end 140.75 61.75) (width 0.2) (layer "F.Cu") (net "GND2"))
 (segment (start 123.25 75.25) (end 123.25 65.25) (width 0.2) (layer "F.Cu") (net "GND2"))
 (segment (start 140.75 61.75) (end 140.75 60.849999) (width 0.2) (layer "F.Cu") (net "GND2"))
 (segment (start 124.46 76.46) (end 123.25 75.25) (width 0.2) (layer "F.Cu") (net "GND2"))
 (segment (start 123.75 64.75) (end 137.75 64.75) (width 0.2) (layer "F.Cu") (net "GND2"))
 (segment (start 102.843198 57.125) (end 119.375 57.125) (width 0.2) (layer "F.Cu") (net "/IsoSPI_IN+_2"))
 (segment (start 140.25 60.099999) (end 140.225 60.074999) (width 0.2) (layer "F.Cu") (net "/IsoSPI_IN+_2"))
 (segment (start 140.225 60.074999) (end 140.225 57.556802) (width 0.2) (layer "F.Cu") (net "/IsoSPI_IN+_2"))
 (segment (start 102.25 60.099999) (end 102.225 60.074999) (width 0.2) (layer "F.Cu") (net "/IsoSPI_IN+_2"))
 (segment (start 102.25 61) (end 102.25 60.099999) (width 0.2) (layer "F.Cu") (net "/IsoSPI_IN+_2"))
 (segment (start 139.343198 56.675) (end 121.675 56.675) (width 0.2) (layer "F.Cu") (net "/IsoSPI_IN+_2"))
 (segment (start 140.25 61) (end 140.25 60.099999) (width 0.2) (layer "F.Cu") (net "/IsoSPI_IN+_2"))
 (segment (start 119.375 57.125) (end 119.75 57.5) (width 0.2) (layer "F.Cu") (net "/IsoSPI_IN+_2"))
 (segment (start 140.225 57.556802) (end 139.343198 56.675) (width 0.2) (layer "F.Cu") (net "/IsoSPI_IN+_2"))
 (segment (start 121.675 56.675) (end 121.25 56.25) (width 0.2) (layer "F.Cu") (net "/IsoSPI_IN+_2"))
 (segment (start 102.225 60.074999) (end 102.225 57.743198) (width 0.2) (layer "F.Cu") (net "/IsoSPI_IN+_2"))
 (segment (start 102.225 57.743198) (end 102.843198 57.125) (width 0.2) (layer "F.Cu") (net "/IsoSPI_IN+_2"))
 (via micro (at 121.25 56.25) (size 0.6) (drill 0.3) (layers "F.Cu" "B.Cu") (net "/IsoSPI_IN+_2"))
 (via micro (at 119.75 57.5) (size 0.6) (drill 0.3) (layers "F.Cu" "B.Cu") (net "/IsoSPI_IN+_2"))
 (segment (start 119.871914 57.5) (end 121.121914 56.25) (width 0.2) (layer "B.Cu") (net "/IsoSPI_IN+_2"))
 (segment (start 119.75 57.5) (end 119.871914 57.5) (width 0.2) (layer "B.Cu") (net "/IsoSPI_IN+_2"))
 (segment (start 121.121914 56.25) (end 121.25 56.25) (width 0.2) (layer "B.Cu") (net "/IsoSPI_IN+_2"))
 (segment (start 139.75 60.099999) (end 139.775 60.074999) (width 0.2) (layer "F.Cu") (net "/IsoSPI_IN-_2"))
 (segment (start 139.156802 57.125) (end 120.875 57.125) (width 0.2) (layer "F.Cu") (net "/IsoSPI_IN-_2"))
 (segment (start 139.775 60.074999) (end 139.775 57.743198) (width 0.2) (layer "F.Cu") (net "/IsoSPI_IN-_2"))
 (segment (start 139.775 57.743198) (end 139.156802 57.125) (width 0.2) (layer "F.Cu") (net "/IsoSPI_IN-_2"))
 (segment (start 139.75 61) (end 139.75 60.099999) (width 0.2) (layer "F.Cu") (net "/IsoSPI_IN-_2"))
 (segment (start 101.775 57.556802) (end 101.775 60.074999) (width 0.2) (layer "F.Cu") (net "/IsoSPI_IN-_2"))
 (segment (start 120.5 56.75) (end 120.425 56.675) (width 0.2) (layer "F.Cu") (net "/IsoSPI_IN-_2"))
 (segment (start 101.75 60.099999) (end 101.75 61) (width 0.2) (layer "F.Cu") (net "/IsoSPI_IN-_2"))
 (segment (start 120.425 56.675) (end 102.656802 56.675) (width 0.2) (layer "F.Cu") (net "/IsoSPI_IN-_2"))
 (segment (start 101.775 60.074999) (end 101.75 60.099999) (width 0.2) (layer "F.Cu") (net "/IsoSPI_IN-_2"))
 (segment (start 102.656802 56.675) (end 101.775 57.556802) (width 0.2) (layer "F.Cu") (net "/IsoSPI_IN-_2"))
 (segment (start 120.875 57.125) (end 120.5 56.75) (width 0.2) (layer "F.Cu") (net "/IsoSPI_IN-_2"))
 (segment (start 101.25 61.75) (end 101.25 60.849999) (width 0.2) (layer "F.Cu") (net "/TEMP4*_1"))
 (segment (start 116.54 69.35) (end 116.54 69.29) (width 0.2) (layer "F.Cu") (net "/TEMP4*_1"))
 (segment (start 116.5 65.25) (end 116 64.75) (width 0.2) (layer "F.Cu") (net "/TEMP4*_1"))
 (segment (start 104.25 64.75) (end 101.25 61.75) (width 0.2) (layer "F.Cu") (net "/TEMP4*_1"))
 (segment (start 116.5 69.25) (end 116.5 65.25) (width 0.2) (layer "F.Cu") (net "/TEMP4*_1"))
 (segment (start 116.54 69.29) (end 116.5 69.25) (width 0.2) (layer "F.Cu") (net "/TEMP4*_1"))
 (segment (start 116 64.75) (end 104.25 64.75) (width 0.2) (layer "F.Cu") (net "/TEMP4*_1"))
 (segment (start 116.54 78.21) (end 116.5 78.25) (width 0.2) (layer "F.Cu") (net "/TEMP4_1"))
 (segment (start 116.54 77.79) (end 116.5 77.75) (width 0.2) (layer "F.Cu") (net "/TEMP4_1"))
 (segment (start 104 65.25) (end 100.75 62) (width 0.2) (layer "F.Cu") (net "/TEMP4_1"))
 (segment (start 100.75 62) (end 100.75 60.85) (width 0.2) (layer "F.Cu") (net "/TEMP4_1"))
 (segment (start 116.5 76.5) (end 115.25 75.25) (width 0.2) (layer "F.Cu") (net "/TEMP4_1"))
 (segment (start 114.75 65.25) (end 104 65.25) (width 0.2) (layer "F.Cu") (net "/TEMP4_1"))
 (segment (start 115.25 75.25) (end 115.25 65.75) (width 0.2) (layer "F.Cu") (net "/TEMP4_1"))
 (segment (start 115.25 65.75) (end 114.75 65.25) (width 0.2) (layer "F.Cu") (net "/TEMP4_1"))
 (segment (start 116.54 78.15) (end 116.54 77.79) (width 0.2) (layer "F.Cu") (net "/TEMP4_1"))
 (segment (start 116.5 77.75) (end 116.5 76.5) (width 0.2) (layer "F.Cu") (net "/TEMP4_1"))
 (segment (start 114 66.25) (end 114 69.35) (width 0.2) (layer "F.Cu") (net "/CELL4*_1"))
 (segment (start 100.25 60.85) (end 100.25 62.25) (width 0.2) (layer "F.Cu") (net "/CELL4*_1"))
 (segment (start 100.25 62.25) (end 103.75 65.75) (width 0.2) (layer "F.Cu") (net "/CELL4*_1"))
 (segment (start 103.75 65.75) (end 113.5 65.75) (width 0.2) (layer "F.Cu") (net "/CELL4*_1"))
 (segment (start 113.5 65.75) (end 114 66.25) (width 0.2) (layer "F.Cu") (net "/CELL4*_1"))
 (segment (start 114 78.15) (end 114 76.5) (width 0.2) (layer "F.Cu") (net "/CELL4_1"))
 (segment (start 112.25 66.25) (end 103.5 66.25) (width 0.2) (layer "F.Cu") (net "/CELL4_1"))
 (segment (start 112.75 66.75) (end 112.25 66.25) (width 0.2) (layer "F.Cu") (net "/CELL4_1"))
 (segment (start 114 76.5) (end 112.75 75.25) (width 0.2) (layer "F.Cu") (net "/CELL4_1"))
 (segment (start 112.75 75.25) (end 112.75 66.75) (width 0.2) (layer "F.Cu") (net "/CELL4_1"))
 (segment (start 99.75 62.5) (end 99.75 60.85) (width 0.2) (layer "F.Cu") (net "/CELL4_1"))
 (segment (start 103.5 66.25) (end 99.75 62.5) (width 0.2) (layer "F.Cu") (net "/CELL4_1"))
 (segment (start 99.25 60.85) (end 99.25 62.75) (width 0.2) (layer "F.Cu") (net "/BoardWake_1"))
 (segment (start 99.25 62.75) (end 103.25 66.75) (width 0.2) (layer "F.Cu") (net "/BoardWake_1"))
 (segment (start 111.46 69.29) (end 111.46 69.35) (width 0.2) (layer "F.Cu") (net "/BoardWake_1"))
 (segment (start 111.5 69.25) (end 111.46 69.29) (width 0.2) (layer "F.Cu") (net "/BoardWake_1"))
 (segment (start 103.25 66.75) (end 111 66.75) (width 0.2) (layer "F.Cu") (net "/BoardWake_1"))
 (segment (start 111 66.75) (end 111.5 67.25) (width 0.2) (layer "F.Cu") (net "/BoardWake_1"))
 (segment (start 111.5 67.25) (end 111.5 69.25) (width 0.2) (layer "F.Cu") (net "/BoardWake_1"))
 (segment (start 111.5 78.11) (end 111.5 76.5) (width 0.2) (layer "F.Cu") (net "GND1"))
 (segment (start 109.75 67.25) (end 103 67.25) (width 0.2) (layer "F.Cu") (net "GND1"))
 (segment (start 98.75 63) (end 98.75 60.849999) (width 0.2) (layer "F.Cu") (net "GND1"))
 (segment (start 110.25 75.25) (end 110.25 67.75) (width 0.2) (layer "F.Cu") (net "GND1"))
 (segment (start 103 67.25) (end 98.75 63) (width 0.2) (layer "F.Cu") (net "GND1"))
 (segment (start 111.46 78.15) (end 111.5 78.11) (width 0.2) (layer "F.Cu") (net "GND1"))
 (segment (start 110.25 67.75) (end 109.75 67.25) (width 0.2) (layer "F.Cu") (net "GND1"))
 (segment (start 111.5 76.5) (end 110.25 75.25) (width 0.2) (layer "F.Cu") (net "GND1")))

